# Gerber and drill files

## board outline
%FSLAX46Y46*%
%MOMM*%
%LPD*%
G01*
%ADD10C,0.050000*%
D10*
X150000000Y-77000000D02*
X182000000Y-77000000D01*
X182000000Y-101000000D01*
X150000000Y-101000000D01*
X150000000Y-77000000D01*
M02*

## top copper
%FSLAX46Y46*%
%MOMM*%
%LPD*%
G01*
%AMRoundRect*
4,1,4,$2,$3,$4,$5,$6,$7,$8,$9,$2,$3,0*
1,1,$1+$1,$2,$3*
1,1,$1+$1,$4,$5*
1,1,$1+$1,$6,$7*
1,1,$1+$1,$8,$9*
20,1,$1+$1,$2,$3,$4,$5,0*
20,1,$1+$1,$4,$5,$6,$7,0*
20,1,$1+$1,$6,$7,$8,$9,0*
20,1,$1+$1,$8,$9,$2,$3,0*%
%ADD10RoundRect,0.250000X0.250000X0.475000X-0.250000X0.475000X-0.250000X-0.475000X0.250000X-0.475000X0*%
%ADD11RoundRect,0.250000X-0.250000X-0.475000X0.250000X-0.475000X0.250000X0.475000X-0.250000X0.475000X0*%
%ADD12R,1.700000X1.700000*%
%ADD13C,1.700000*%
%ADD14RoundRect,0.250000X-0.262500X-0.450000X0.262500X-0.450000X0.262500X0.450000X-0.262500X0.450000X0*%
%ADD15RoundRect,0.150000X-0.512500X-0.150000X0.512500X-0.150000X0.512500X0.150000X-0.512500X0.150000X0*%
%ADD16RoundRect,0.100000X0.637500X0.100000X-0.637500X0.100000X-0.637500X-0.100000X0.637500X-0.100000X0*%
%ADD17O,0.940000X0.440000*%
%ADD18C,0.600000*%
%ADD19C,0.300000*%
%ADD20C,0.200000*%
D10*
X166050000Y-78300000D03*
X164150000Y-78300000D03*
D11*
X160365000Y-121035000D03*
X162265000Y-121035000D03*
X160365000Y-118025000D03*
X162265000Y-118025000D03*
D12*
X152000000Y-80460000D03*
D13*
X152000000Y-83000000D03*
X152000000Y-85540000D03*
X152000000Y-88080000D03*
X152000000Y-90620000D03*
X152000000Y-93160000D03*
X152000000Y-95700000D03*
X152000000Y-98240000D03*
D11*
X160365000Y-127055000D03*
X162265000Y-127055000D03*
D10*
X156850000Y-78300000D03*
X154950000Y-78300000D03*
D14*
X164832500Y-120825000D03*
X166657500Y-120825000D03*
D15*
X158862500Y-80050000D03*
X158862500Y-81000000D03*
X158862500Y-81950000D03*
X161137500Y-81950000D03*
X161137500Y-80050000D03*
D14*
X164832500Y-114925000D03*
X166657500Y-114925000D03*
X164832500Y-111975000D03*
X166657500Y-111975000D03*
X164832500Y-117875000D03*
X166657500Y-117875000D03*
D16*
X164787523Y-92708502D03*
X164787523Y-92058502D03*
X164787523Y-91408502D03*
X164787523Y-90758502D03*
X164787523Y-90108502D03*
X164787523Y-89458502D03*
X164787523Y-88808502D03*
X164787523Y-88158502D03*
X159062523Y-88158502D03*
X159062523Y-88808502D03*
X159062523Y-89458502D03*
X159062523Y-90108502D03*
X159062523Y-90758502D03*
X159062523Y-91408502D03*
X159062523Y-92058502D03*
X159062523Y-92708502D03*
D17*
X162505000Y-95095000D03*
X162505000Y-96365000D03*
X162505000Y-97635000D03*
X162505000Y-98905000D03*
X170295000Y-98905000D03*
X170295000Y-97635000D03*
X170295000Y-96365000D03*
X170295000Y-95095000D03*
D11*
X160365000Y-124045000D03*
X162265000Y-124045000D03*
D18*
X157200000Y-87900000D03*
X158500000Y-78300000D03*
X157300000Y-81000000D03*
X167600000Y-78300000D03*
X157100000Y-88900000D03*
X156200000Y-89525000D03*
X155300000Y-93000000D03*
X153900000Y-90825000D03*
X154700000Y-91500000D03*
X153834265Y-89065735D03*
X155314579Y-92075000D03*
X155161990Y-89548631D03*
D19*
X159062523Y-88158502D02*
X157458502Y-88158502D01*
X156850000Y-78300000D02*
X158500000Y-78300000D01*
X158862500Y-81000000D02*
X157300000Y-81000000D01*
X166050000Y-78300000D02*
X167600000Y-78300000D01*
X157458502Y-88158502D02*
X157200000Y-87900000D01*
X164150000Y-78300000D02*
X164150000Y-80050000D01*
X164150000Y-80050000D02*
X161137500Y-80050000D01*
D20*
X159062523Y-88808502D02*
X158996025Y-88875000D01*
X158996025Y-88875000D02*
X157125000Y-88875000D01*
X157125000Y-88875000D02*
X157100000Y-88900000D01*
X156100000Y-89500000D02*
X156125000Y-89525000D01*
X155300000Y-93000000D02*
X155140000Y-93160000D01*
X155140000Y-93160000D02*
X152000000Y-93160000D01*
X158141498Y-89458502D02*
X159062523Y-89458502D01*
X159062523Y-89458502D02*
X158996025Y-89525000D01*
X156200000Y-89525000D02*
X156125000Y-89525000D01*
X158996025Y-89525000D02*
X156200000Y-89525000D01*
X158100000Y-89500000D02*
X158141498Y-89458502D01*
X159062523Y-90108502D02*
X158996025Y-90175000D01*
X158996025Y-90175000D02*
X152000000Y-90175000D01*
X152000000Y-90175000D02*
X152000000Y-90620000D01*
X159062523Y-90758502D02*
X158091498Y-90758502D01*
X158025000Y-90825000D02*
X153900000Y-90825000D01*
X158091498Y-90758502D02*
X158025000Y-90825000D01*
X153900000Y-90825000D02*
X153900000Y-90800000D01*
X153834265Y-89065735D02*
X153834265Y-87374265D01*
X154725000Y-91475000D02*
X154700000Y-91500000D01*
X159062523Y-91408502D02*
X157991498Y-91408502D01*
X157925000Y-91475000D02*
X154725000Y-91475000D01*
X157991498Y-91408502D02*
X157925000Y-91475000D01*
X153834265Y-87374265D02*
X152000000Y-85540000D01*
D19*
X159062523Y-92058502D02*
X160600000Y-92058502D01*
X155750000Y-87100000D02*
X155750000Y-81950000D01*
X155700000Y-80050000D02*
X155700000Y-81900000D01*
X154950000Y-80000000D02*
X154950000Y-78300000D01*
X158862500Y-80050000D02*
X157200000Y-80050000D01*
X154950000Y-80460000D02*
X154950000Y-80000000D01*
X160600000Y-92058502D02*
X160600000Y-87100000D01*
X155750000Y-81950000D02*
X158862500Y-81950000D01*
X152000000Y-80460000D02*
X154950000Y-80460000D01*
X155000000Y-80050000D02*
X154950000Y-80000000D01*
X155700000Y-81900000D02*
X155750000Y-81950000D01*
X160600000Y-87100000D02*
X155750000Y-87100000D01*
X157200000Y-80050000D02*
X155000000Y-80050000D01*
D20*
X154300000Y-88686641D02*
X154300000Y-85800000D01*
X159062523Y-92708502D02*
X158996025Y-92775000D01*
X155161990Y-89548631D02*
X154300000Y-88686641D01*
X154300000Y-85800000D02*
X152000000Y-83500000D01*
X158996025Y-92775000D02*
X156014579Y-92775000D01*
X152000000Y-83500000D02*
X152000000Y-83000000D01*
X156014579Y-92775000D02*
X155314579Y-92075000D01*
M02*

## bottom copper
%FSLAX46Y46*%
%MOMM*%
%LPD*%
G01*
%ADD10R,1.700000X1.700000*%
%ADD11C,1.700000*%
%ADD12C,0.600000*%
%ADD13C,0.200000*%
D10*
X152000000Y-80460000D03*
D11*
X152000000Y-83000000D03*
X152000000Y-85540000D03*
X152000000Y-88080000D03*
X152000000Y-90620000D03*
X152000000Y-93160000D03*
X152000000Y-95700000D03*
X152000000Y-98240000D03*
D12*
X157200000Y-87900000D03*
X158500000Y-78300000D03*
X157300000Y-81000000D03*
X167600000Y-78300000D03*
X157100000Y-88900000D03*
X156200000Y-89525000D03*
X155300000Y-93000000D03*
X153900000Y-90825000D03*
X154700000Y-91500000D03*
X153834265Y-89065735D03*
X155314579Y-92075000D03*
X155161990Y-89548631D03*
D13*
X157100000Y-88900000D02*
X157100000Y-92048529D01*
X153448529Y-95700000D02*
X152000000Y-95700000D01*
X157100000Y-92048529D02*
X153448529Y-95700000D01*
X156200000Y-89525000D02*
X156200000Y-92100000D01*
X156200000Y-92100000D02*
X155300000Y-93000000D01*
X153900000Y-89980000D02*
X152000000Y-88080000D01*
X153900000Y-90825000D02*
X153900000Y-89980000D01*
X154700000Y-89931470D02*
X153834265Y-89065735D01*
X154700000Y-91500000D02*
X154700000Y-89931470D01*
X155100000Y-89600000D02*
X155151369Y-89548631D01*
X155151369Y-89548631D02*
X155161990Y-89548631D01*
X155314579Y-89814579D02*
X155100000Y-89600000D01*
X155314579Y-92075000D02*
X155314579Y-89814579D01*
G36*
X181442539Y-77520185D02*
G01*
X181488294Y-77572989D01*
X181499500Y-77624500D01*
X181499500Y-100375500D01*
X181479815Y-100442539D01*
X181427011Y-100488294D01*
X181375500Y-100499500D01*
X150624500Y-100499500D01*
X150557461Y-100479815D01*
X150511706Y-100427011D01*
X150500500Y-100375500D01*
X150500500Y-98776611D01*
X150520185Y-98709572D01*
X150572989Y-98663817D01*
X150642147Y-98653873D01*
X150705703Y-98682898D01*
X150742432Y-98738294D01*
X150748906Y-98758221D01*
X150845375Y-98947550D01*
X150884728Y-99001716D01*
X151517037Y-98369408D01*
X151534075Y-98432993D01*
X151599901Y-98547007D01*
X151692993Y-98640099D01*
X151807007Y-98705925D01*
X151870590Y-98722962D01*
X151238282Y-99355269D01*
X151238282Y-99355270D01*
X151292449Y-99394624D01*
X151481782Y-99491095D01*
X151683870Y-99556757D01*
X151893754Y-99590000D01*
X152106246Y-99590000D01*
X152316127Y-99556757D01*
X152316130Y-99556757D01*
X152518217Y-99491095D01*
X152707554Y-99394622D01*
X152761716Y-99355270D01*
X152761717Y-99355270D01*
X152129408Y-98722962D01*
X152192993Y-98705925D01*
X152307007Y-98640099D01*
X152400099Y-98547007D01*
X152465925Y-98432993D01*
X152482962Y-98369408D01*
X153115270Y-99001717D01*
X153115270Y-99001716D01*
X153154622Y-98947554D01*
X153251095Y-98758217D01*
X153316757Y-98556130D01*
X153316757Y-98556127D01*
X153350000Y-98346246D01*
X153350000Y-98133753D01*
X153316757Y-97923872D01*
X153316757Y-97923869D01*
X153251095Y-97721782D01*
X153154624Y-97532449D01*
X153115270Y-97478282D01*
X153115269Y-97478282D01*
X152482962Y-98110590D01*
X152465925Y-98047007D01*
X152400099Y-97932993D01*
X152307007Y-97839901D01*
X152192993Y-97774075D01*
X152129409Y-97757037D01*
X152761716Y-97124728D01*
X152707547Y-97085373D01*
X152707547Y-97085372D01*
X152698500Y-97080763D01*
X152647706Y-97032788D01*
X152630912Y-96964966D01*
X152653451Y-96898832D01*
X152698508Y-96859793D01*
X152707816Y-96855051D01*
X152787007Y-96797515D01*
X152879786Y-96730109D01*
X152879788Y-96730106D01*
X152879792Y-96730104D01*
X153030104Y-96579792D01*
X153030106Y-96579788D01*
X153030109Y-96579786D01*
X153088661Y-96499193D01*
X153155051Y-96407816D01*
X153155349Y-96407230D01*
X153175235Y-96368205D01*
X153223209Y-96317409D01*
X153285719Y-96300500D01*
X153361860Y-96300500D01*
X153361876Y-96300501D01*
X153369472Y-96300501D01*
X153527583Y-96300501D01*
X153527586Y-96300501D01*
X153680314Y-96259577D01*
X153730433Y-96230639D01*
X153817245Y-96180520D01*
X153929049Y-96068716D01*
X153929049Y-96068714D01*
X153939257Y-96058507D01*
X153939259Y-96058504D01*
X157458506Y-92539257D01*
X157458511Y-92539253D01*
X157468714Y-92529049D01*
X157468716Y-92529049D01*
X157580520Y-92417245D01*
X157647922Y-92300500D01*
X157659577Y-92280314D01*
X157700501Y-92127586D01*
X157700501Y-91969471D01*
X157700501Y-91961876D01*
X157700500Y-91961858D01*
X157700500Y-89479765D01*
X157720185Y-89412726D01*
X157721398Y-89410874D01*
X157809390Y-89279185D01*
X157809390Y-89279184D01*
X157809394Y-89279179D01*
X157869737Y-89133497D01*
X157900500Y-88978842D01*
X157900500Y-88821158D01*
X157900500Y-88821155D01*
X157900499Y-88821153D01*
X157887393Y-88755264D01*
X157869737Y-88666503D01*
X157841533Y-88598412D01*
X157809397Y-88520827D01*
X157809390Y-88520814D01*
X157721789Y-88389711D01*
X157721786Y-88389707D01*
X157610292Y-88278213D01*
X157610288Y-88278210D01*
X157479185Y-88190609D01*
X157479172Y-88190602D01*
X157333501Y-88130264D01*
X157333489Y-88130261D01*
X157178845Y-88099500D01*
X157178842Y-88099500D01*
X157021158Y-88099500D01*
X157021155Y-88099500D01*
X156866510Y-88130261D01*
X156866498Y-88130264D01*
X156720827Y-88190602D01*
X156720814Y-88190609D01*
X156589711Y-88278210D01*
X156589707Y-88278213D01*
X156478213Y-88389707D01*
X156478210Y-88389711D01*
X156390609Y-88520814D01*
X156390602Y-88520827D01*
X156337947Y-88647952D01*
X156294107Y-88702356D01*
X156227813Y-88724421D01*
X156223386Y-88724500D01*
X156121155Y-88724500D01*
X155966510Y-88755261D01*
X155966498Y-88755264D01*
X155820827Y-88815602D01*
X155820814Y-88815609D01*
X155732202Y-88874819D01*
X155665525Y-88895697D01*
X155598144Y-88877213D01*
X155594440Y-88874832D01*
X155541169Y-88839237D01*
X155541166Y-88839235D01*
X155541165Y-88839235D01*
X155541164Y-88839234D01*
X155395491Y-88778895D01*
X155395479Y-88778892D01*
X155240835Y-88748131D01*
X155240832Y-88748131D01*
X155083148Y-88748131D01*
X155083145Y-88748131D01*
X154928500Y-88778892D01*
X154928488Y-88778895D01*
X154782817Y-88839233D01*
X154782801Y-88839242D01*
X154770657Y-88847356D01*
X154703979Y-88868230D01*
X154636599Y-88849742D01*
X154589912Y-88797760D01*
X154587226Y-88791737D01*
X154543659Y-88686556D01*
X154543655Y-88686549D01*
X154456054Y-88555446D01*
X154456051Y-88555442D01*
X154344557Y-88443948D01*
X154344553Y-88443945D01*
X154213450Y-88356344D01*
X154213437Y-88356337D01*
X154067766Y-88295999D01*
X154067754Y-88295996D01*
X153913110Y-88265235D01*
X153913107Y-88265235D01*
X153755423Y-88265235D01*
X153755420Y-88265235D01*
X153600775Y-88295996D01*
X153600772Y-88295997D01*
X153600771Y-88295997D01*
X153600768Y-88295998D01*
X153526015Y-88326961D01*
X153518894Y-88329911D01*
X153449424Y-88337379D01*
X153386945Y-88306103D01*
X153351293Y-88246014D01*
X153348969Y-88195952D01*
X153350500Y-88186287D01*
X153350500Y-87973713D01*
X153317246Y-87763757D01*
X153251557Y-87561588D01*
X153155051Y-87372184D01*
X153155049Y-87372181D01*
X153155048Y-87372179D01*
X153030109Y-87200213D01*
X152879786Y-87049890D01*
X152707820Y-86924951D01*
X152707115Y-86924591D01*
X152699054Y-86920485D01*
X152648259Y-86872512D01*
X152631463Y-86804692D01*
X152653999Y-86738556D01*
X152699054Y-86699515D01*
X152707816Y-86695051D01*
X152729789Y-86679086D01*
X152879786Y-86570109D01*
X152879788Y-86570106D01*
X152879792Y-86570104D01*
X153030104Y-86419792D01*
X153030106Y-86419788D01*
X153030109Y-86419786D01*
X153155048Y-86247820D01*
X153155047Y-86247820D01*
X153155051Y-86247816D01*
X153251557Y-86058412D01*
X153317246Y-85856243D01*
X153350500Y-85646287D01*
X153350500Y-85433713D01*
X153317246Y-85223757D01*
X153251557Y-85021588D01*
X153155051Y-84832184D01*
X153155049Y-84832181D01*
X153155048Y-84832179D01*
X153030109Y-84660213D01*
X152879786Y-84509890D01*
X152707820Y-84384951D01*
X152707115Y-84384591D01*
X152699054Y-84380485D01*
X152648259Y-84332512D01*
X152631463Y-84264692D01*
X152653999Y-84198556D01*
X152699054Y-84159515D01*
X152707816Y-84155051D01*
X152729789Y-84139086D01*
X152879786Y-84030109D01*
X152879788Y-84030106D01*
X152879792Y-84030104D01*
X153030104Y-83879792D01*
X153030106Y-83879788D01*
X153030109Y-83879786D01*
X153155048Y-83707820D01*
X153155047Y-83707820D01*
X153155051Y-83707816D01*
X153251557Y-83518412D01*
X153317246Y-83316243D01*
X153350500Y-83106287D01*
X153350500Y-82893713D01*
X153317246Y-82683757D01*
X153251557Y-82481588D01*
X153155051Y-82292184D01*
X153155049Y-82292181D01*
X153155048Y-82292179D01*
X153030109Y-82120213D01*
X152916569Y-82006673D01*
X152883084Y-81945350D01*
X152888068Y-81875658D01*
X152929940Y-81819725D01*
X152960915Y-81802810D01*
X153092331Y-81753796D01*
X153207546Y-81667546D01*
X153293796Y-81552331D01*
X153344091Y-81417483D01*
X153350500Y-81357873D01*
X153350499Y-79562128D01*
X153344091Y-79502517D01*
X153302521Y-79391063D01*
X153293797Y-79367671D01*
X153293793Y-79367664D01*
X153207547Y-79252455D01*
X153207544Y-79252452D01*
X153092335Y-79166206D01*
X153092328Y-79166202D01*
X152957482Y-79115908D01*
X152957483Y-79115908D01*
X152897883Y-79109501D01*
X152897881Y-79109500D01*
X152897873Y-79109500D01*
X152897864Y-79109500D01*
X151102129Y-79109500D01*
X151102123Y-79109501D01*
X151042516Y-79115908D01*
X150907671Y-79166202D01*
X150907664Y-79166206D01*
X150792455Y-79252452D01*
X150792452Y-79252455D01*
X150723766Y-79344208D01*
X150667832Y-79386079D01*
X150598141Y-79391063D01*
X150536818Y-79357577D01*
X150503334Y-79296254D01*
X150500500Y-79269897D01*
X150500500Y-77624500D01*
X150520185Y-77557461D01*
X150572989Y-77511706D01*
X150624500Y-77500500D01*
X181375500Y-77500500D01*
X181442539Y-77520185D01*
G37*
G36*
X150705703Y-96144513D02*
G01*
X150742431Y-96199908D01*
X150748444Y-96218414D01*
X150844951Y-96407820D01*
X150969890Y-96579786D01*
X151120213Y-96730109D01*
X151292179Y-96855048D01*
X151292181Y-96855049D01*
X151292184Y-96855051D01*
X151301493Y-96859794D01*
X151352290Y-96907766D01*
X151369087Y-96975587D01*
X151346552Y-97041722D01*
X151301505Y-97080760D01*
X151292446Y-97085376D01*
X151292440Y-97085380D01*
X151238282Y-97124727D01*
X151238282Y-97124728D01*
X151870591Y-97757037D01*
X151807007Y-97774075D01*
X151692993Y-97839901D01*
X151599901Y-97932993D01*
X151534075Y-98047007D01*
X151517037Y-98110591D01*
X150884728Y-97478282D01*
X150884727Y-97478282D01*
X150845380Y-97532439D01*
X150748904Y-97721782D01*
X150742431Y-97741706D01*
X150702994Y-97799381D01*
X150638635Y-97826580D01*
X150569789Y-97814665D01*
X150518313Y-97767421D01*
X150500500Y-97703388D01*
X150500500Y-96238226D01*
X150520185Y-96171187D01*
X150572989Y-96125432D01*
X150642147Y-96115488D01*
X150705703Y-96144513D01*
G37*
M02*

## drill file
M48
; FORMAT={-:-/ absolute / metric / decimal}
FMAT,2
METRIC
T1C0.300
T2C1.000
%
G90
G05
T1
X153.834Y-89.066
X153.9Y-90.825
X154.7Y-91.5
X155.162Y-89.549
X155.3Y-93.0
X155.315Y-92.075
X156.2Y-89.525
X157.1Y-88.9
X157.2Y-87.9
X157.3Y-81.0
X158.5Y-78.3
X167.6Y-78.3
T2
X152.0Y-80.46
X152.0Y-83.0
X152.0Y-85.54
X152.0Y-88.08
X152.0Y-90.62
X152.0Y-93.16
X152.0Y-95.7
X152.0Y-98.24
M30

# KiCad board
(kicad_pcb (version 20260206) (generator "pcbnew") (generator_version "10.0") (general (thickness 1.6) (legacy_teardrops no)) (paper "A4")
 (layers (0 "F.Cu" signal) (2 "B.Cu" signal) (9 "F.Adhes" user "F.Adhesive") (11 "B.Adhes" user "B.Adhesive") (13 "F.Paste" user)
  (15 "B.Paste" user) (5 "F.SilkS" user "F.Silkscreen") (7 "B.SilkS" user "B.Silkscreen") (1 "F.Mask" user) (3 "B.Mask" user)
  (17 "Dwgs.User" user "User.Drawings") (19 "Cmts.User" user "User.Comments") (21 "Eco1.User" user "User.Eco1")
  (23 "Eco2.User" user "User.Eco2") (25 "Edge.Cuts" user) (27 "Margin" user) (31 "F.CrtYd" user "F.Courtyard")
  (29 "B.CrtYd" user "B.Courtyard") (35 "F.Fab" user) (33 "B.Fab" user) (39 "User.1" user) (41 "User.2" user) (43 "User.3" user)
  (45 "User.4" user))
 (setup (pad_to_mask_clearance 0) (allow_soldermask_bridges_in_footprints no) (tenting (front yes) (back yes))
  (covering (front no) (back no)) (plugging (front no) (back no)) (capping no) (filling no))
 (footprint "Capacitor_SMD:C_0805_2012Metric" (layer "F.Cu") (at 165.1 78.3 180)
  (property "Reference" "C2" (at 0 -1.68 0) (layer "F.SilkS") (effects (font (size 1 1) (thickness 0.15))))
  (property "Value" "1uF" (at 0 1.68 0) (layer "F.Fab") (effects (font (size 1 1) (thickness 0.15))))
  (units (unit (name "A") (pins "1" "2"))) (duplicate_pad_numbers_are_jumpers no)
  (pad "1" smd roundrect (at -0.95 0 180) (size 1 1.45) (layers "F.Cu" "F.Mask" "F.Paste") (roundrect_rratio 0.25) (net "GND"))
  (pad "2" smd roundrect (at 0.95 0 180) (size 1 1.45) (layers "F.Cu" "F.Mask" "F.Paste") (roundrect_rratio 0.25) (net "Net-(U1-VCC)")))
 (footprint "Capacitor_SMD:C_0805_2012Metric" (layer "F.Cu") (at 161.315 121.035)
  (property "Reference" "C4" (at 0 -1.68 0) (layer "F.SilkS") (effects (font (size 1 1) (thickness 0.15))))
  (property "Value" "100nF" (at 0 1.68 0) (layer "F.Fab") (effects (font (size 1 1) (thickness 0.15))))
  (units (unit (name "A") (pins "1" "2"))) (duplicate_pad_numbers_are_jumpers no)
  (pad "1" smd roundrect (at -0.95 0) (size 1 1.45) (layers "F.Cu" "F.Mask" "F.Paste") (roundrect_rratio 0.25) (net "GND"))
  (pad "2" smd roundrect (at 0.95 0) (size 1 1.45) (layers "F.Cu" "F.Mask" "F.Paste") (roundrect_rratio 0.25) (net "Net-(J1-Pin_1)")))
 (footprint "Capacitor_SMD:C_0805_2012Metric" (layer "F.Cu") (at 161.315 118.025)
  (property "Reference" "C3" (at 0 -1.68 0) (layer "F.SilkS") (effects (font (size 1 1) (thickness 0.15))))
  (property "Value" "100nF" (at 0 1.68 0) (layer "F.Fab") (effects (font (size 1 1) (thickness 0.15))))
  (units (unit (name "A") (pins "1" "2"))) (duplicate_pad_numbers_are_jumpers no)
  (pad "1" smd roundrect (at -0.95 0) (size 1 1.45) (layers "F.Cu" "F.Mask" "F.Paste") (roundrect_rratio 0.25) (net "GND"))
  (pad "2" smd roundrect (at 0.95 0) (size 1 1.45) (layers "F.Cu" "F.Mask" "F.Paste") (roundrect_rratio 0.25) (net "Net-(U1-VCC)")))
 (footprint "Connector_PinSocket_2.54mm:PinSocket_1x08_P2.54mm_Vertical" (layer "F.Cu") (at 152 80.46)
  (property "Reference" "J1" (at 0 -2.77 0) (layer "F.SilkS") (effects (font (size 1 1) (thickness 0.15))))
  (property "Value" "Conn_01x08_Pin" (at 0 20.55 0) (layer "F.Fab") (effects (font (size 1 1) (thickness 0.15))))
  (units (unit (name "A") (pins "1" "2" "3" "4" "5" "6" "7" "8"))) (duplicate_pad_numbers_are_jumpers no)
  (pad "1" thru_hole rect (at 0 0) (size 1.7 1.7) (drill 1) (layers "*.Cu" "*.Mask") (remove_unused_layers no) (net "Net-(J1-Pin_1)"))
  (pad "2" thru_hole circle (at 0 2.54) (size 1.7 1.7) (drill 1) (layers "*.Cu" "*.Mask") (remove_unused_layers no) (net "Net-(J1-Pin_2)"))
  (pad "3" thru_hole circle (at 0 5.08) (size 1.7 1.7) (drill 1) (layers "*.Cu" "*.Mask") (remove_unused_layers no) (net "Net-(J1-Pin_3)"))
  (pad "4" thru_hole circle (at 0 7.62) (size 1.7 1.7) (drill 1) (layers "*.Cu" "*.Mask") (remove_unused_layers no) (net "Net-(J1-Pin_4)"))
  (pad "5" thru_hole circle (at 0 10.16) (size 1.7 1.7) (drill 1) (layers "*.Cu" "*.Mask") (remove_unused_layers no) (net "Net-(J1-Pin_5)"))
  (pad "6" thru_hole circle (at 0 12.7) (size 1.7 1.7) (drill 1) (layers "*.Cu" "*.Mask") (remove_unused_layers no) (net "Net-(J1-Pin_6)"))
  (pad "7" thru_hole circle (at 0 15.24) (size 1.7 1.7) (drill 1) (layers "*.Cu" "*.Mask") (remove_unused_layers no) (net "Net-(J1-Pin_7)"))
  (pad "8" thru_hole circle (at 0 17.78) (size 1.7 1.7) (drill 1) (layers "*.Cu" "*.Mask") (remove_unused_layers no) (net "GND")))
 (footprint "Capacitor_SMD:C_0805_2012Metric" (layer "F.Cu") (at 161.315 127.055)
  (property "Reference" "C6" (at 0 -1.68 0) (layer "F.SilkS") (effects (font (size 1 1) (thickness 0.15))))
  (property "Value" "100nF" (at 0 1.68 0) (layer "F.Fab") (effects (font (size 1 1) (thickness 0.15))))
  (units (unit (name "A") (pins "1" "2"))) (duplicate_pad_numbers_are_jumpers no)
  (pad "1" smd roundrect (at -0.95 0) (size 1 1.45) (layers "F.Cu" "F.Mask" "F.Paste") (roundrect_rratio 0.25) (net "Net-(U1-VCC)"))
  (pad "2" smd roundrect (at 0.95 0) (size 1 1.45) (layers "F.Cu" "F.Mask" "F.Paste") (roundrect_rratio 0.25) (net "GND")))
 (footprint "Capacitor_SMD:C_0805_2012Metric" (layer "F.Cu") (at 155.9 78.3 180)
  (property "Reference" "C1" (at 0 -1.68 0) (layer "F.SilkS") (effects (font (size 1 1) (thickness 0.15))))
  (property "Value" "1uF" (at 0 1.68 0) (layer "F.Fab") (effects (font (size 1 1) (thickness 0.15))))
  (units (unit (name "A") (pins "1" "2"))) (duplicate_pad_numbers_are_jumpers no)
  (pad "1" smd roundrect (at -0.95 0 180) (size 1 1.45) (layers "F.Cu" "F.Mask" "F.Paste") (roundrect_rratio 0.25) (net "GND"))
  (pad "2" smd roundrect (at 0.95 0 180) (size 1 1.45) (layers "F.Cu" "F.Mask" "F.Paste") (roundrect_rratio 0.25) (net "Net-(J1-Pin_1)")))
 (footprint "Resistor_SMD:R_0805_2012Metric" (layer "F.Cu") (at 165.745 120.825)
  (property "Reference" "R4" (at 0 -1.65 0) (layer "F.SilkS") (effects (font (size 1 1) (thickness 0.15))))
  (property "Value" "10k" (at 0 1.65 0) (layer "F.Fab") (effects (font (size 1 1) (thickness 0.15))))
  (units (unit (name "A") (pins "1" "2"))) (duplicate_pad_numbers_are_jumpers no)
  (pad "1" smd roundrect (at -0.9125 0) (size 1.025 1.4) (layers "F.Cu" "F.Mask" "F.Paste") (roundrect_rratio 0.243902) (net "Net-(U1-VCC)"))
  (pad "2" smd roundrect (at 0.9125 0) (size 1.025 1.4) (layers "F.Cu" "F.Mask" "F.Paste") (roundrect_rratio 0.243902)
   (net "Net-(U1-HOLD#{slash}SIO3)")))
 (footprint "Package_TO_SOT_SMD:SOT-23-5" (layer "F.Cu") (at 160 81)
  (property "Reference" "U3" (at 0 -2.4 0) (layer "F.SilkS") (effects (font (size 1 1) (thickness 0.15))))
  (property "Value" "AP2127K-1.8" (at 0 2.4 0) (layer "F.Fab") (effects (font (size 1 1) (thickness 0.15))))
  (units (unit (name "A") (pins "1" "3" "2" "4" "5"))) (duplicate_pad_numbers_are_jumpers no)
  (pad "1" smd roundrect (at -1.1375 -0.95) (size 1.325 0.6) (layers "F.Cu" "F.Mask" "F.Paste") (roundrect_rratio 0.25)
   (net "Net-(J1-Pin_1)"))
  (pad "2" smd roundrect (at -1.1375 0) (size 1.325 0.6) (layers "F.Cu" "F.Mask" "F.Paste") (roundrect_rratio 0.25) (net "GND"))
  (pad "3" smd roundrect (at -1.1375 0.95) (size 1.325 0.6) (layers "F.Cu" "F.Mask" "F.Paste") (roundrect_rratio 0.25)
   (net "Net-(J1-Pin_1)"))
  (pad "4" smd roundrect (at 1.1375 0.95) (size 1.325 0.6) (layers "F.Cu" "F.Mask" "F.Paste") (roundrect_rratio 0.25)
   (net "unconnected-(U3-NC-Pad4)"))
  (pad "5" smd roundrect (at 1.1375 -0.95) (size 1.325 0.6) (layers "F.Cu" "F.Mask" "F.Paste") (roundrect_rratio 0.25) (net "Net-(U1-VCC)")))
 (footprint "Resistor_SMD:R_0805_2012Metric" (layer "F.Cu") (at 165.745 114.925)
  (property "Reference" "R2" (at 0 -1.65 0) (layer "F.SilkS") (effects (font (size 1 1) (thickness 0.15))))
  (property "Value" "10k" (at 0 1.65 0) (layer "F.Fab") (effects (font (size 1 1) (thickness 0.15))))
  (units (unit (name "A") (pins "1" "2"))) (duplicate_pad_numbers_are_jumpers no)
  (pad "1" smd roundrect (at -0.9125 0) (size 1.025 1.4) (layers "F.Cu" "F.Mask" "F.Paste") (roundrect_rratio 0.243902) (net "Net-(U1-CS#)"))
  (pad "2" smd roundrect (at 0.9125 0) (size 1.025 1.4) (layers "F.Cu" "F.Mask" "F.Paste") (roundrect_rratio 0.243902) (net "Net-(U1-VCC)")))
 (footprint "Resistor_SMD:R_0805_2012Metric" (layer "F.Cu") (at 165.745 111.975)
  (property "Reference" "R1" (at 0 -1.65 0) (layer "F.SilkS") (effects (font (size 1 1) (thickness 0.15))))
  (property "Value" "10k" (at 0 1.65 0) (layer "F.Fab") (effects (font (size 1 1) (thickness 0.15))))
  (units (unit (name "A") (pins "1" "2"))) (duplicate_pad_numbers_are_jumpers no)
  (pad "1" smd roundrect (at -0.9125 0) (size 1.025 1.4) (layers "F.Cu" "F.Mask" "F.Paste") (roundrect_rratio 0.243902) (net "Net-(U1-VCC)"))
  (pad "2" smd roundrect (at 0.9125 0) (size 1.025 1.4) (layers "F.Cu" "F.Mask" "F.Paste") (roundrect_rratio 0.243902) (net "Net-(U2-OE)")))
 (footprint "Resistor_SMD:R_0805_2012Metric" (layer "F.Cu") (at 165.745 117.875)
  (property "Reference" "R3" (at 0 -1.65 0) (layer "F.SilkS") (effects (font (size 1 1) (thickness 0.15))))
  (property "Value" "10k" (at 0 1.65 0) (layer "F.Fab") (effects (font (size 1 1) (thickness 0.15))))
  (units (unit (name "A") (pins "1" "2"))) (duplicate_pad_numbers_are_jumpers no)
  (pad "1" smd roundrect (at -0.9125 0) (size 1.025 1.4) (layers "F.Cu" "F.Mask" "F.Paste") (roundrect_rratio 0.243902) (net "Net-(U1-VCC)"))
  (pad "2" smd roundrect (at 0.9125 0) (size 1.025 1.4) (layers "F.Cu" "F.Mask" "F.Paste") (roundrect_rratio 0.243902)
   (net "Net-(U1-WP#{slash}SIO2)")))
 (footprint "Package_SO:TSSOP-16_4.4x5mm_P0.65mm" (layer "F.Cu") (at 161.925023 90.433502 180)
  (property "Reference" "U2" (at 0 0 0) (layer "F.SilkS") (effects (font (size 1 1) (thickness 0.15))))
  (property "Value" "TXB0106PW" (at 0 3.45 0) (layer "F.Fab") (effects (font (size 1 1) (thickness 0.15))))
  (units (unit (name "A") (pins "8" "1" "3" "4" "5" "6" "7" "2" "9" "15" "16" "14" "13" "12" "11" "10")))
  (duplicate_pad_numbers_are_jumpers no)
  (pad "1" smd roundrect (at -2.8625 -2.275 180) (size 1.475 0.4) (layers "F.Cu" "F.Mask" "F.Paste") (roundrect_rratio 0.25)
   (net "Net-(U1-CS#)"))
  (pad "2" smd roundrect (at -2.8625 -1.625 180) (size 1.475 0.4) (layers "F.Cu" "F.Mask" "F.Paste") (roundrect_rratio 0.25)
   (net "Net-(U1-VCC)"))
  (pad "3" smd roundrect (at -2.8625 -0.975 180) (size 1.475 0.4) (layers "F.Cu" "F.Mask" "F.Paste") (roundrect_rratio 0.25)
   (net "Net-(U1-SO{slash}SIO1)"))
  (pad "4" smd roundrect (at -2.8625 -0.325 180) (size 1.475 0.4) (layers "F.Cu" "F.Mask" "F.Paste") (roundrect_rratio 0.25)
   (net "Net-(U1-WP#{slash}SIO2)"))
  (pad "5" smd roundrect (at -2.8625 0.325 180) (size 1.475 0.4) (layers "F.Cu" "F.Mask" "F.Paste") (roundrect_rratio 0.25)
   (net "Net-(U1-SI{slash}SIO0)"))
  (pad "6" smd roundrect (at -2.8625 0.975 180) (size 1.475 0.4) (layers "F.Cu" "F.Mask" "F.Paste") (roundrect_rratio 0.25)
   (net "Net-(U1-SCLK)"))
  (pad "7" smd roundrect (at -2.8625 1.625 180) (size 1.475 0.4) (layers "F.Cu" "F.Mask" "F.Paste") (roundrect_rratio 0.25)
   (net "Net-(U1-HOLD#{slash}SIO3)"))
  (pad "8" smd roundrect (at -2.8625 2.275 180) (size 1.475 0.4) (layers "F.Cu" "F.Mask" "F.Paste") (roundrect_rratio 0.25)
   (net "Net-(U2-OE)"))
  (pad "9" smd roundrect (at 2.8625 2.275 180) (size 1.475 0.4) (layers "F.Cu" "F.Mask" "F.Paste") (roundrect_rratio 0.25) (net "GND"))
  (pad "10" smd roundrect (at 2.8625 1.625 180) (size 1.475 0.4) (layers "F.Cu" "F.Mask" "F.Paste") (roundrect_rratio 0.25)
   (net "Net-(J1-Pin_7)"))
  (pad "11" smd roundrect (at 2.8625 0.975 180) (size 1.475 0.4) (layers "F.Cu" "F.Mask" "F.Paste") (roundrect_rratio 0.25)
   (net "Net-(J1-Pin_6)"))
  (pad "12" smd roundrect (at 2.8625 0.325 180) (size 1.475 0.4) (layers "F.Cu" "F.Mask" "F.Paste") (roundrect_rratio 0.25)
   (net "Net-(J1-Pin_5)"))
  (pad "13" smd roundrect (at 2.8625 -0.325 180) (size 1.475 0.4) (layers "F.Cu" "F.Mask" "F.Paste") (roundrect_rratio 0.25)
   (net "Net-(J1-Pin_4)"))
  (pad "14" smd roundrect (at 2.8625 -0.975 180) (size 1.475 0.4) (layers "F.Cu" "F.Mask" "F.Paste") (roundrect_rratio 0.25)
   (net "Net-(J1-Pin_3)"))
  (pad "15" smd roundrect (at 2.8625 -1.625 180) (size 1.475 0.4) (layers "F.Cu" "F.Mask" "F.Paste") (roundrect_rratio 0.25)
   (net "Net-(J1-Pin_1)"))
  (pad "16" smd roundrect (at 2.8625 -2.275 180) (size 1.475 0.4) (layers "F.Cu" "F.Mask" "F.Paste") (roundrect_rratio 0.25)
   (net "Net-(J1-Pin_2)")))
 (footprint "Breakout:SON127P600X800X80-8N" (layer "F.Cu") (at 166.4 97)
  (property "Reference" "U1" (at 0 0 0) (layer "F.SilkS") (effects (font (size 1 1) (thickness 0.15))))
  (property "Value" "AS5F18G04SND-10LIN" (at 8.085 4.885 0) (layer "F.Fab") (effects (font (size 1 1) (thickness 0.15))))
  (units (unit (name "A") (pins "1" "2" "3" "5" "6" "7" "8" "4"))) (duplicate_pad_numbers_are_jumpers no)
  (pad "1" smd oval (at -3.895 -1.905) (size 0.94 0.44) (layers "F.Cu" "F.Mask" "F.Paste") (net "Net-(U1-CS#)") (solder_mask_margin 0.102))
  (pad "2" smd oval (at -3.895 -0.635) (size 0.94 0.44) (layers "F.Cu" "F.Mask" "F.Paste") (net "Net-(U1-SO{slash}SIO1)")
   (solder_mask_margin 0.102))
  (pad "3" smd oval (at -3.895 0.635) (size 0.94 0.44) (layers "F.Cu" "F.Mask" "F.Paste") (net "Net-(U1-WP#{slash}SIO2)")
   (solder_mask_margin 0.102))
  (pad "4" smd oval (at -3.895 1.905) (size 0.94 0.44) (layers "F.Cu" "F.Mask" "F.Paste") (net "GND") (solder_mask_margin 0.102))
  (pad "5" smd oval (at 3.895 1.905) (size 0.94 0.44) (layers "F.Cu" "F.Mask" "F.Paste") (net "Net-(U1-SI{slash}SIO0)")
   (solder_mask_margin 0.102))
  (pad "6" smd oval (at 3.895 0.635) (size 0.94 0.44) (layers "F.Cu" "F.Mask" "F.Paste") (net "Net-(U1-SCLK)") (solder_mask_margin 0.102))
  (pad "7" smd oval (at 3.895 -0.635) (size 0.94 0.44) (layers "F.Cu" "F.Mask" "F.Paste") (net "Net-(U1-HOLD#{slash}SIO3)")
   (solder_mask_margin 0.102))
  (pad "8" smd oval (at 3.895 -1.905) (size 0.94 0.44) (layers "F.Cu" "F.Mask" "F.Paste") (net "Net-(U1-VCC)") (solder_mask_margin 0.102)))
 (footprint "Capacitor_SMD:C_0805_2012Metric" (layer "F.Cu") (at 161.315 124.045)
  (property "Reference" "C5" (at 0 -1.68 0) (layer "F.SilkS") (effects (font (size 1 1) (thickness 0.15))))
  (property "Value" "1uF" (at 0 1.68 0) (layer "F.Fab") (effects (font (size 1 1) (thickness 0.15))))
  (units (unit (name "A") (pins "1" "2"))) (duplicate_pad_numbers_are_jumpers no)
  (pad "1" smd roundrect (at -0.95 0) (size 1 1.45) (layers "F.Cu" "F.Mask" "F.Paste") (roundrect_rratio 0.25) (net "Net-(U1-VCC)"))
  (pad "2" smd roundrect (at 0.95 0) (size 1 1.45) (layers "F.Cu" "F.Mask" "F.Paste") (roundrect_rratio 0.25) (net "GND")))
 (gr_rect (start 150 77) (end 182 101) (stroke (width 0.05) (type default)) (fill no) (layer "Edge.Cuts"))
 (segment (start 159.062523 88.158502) (end 157.458502 88.158502) (width 0.3) (layer "F.Cu") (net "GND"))
 (segment (start 156.85 78.3) (end 158.5 78.3) (width 0.3) (layer "F.Cu") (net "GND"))
 (segment (start 158.8625 81) (end 157.3 81) (width 0.3) (layer "F.Cu") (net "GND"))
 (segment (start 166.05 78.3) (end 167.6 78.3) (width 0.3) (layer "F.Cu") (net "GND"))
 (segment (start 157.458502 88.158502) (end 157.2 87.9) (width 0.3) (layer "F.Cu") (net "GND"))
 (via (at 157.2 87.9) (size 0.6) (drill 0.3) (layers "F.Cu" "B.Cu") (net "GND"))
 (via (at 158.5 78.3) (size 0.6) (drill 0.3) (layers "F.Cu" "B.Cu") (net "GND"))
 (via (at 157.3 81) (size 0.6) (drill 0.3) (layers "F.Cu" "B.Cu") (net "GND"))
 (via (at 167.6 78.3) (size 0.6) (drill 0.3) (layers "F.Cu" "B.Cu") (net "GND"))
 (segment (start 164.15 78.3) (end 164.15 80.05) (width 0.3) (layer "F.Cu") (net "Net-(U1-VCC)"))
 (segment (start 164.15 80.05) (end 161.1375 80.05) (width 0.3) (layer "F.Cu") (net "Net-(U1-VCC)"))
 (segment (start 159.062523 88.808502) (end 158.996025 88.875) (width 0.2) (layer "F.Cu") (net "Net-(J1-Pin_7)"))
 (segment (start 158.996025 88.875) (end 157.125 88.875) (width 0.2) (layer "F.Cu") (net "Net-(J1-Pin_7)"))
 (segment (start 157.125 88.875) (end 157.1 88.9) (width 0.2) (layer "F.Cu") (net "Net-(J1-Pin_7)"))
 (via (at 157.1 88.9) (size 0.6) (drill 0.3) (layers "F.Cu" "B.Cu") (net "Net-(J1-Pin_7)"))
 (segment (start 157.1 88.9) (end 157.1 92.048529) (width 0.2) (layer "B.Cu") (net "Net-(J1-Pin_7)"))
 (segment (start 153.448529 95.7) (end 152 95.7) (width 0.2) (layer "B.Cu") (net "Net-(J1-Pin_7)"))
 (segment (start 157.1 92.048529) (end 153.448529 95.7) (width 0.2) (layer "B.Cu") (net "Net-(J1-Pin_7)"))
 (segment (start 156.1 89.5) (end 156.125 89.525) (width 0.2) (layer "F.Cu") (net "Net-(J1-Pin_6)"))
 (segment (start 155.3 93) (end 155.14 93.16) (width 0.2) (layer "F.Cu") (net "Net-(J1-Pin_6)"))
 (segment (start 155.14 93.16) (end 152 93.16) (width 0.2) (layer "F.Cu") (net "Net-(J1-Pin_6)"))
 (segment (start 158.141498 89.458502) (end 159.062523 89.458502) (width 0.2) (layer "F.Cu") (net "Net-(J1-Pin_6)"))
 (segment (start 159.062523 89.458502) (end 158.996025 89.525) (width 0.2) (layer "F.Cu") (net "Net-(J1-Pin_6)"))
 (segment (start 156.2 89.525) (end 156.125 89.525) (width 0.2) (layer "F.Cu") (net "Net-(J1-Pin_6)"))
 (segment (start 158.996025 89.525) (end 156.2 89.525) (width 0.2) (layer "F.Cu") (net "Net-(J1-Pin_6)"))
 (segment (start 158.1 89.5) (end 158.141498 89.458502) (width 0.2) (layer "F.Cu") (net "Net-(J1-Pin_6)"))
 (via (at 156.2 89.525) (size 0.6) (drill 0.3) (layers "F.Cu" "B.Cu") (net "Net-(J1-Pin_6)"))
 (via (at 155.3 93) (size 0.6) (drill 0.3) (layers "F.Cu" "B.Cu") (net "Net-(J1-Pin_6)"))
 (segment (start 156.2 89.525) (end 156.2 92.1) (width 0.2) (layer "B.Cu") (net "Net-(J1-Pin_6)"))
 (segment (start 156.2 92.1) (end 155.3 93) (width 0.2) (layer "B.Cu") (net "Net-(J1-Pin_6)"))
 (segment (start 159.062523 90.108502) (end 158.996025 90.175) (width 0.2) (layer "F.Cu") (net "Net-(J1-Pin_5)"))
 (segment (start 158.996025 90.175) (end 152 90.175) (width 0.2) (layer "F.Cu") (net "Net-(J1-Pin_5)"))
 (segment (start 152 90.175) (end 152 90.62) (width 0.2) (layer "F.Cu") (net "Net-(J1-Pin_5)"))
 (segment (start 159.062523 90.758502) (end 158.091498 90.758502) (width 0.2) (layer "F.Cu") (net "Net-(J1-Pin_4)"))
 (segment (start 158.025 90.825) (end 153.9 90.825) (width 0.2) (layer "F.Cu") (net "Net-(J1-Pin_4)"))
 (segment (start 158.091498 90.758502) (end 158.025 90.825) (width 0.2) (layer "F.Cu") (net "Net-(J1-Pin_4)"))
 (segment (start 153.9 90.825) (end 153.9 90.8) (width 0.2) (layer "F.Cu") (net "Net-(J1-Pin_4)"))
 (via (at 153.9 90.825) (size 0.6) (drill 0.3) (layers "F.Cu" "B.Cu") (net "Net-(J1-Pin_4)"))
 (segment (start 153.9 89.98) (end 152 88.08) (width 0.2) (layer "B.Cu") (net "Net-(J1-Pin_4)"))
 (segment (start 153.9 90.825) (end 153.9 89.98) (width 0.2) (layer "B.Cu") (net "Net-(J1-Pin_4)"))
 (segment (start 153.834265 89.065735) (end 153.834265 87.374265) (width 0.2) (layer "F.Cu") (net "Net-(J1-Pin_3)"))
 (segment (start 154.725 91.475) (end 154.7 91.5) (width 0.2) (layer "F.Cu") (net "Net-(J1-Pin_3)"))
 (segment (start 159.062523 91.408502) (end 157.991498 91.408502) (width 0.2) (layer "F.Cu") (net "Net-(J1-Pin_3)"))
 (segment (start 157.925 91.475) (end 154.725 91.475) (width 0.2) (layer "F.Cu") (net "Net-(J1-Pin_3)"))
 (segment (start 157.991498 91.408502) (end 157.925 91.475) (width 0.2) (layer "F.Cu") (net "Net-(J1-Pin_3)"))
 (segment (start 153.834265 87.374265) (end 152 85.54) (width 0.2) (layer "F.Cu") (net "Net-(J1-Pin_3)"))
 (via (at 154.7 91.5) (size 0.6) (drill 0.3) (layers "F.Cu" "B.Cu") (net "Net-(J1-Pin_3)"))
 (via (at 153.834265 89.065735) (size 0.6) (drill 0.3) (layers "F.Cu" "B.Cu") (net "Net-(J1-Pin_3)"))
 (segment (start 154.7 89.93147) (end 153.834265 89.065735) (width 0.2) (layer "B.Cu") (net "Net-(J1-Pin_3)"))
 (segment (start 154.7 91.5) (end 154.7 89.93147) (width 0.2) (layer "B.Cu") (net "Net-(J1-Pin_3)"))
 (segment (start 159.062523 92.058502) (end 160.6 92.058502) (width 0.3) (layer "F.Cu") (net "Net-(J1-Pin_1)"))
 (segment (start 155.75 87.1) (end 155.75 81.95) (width 0.3) (layer "F.Cu") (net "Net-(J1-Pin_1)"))
 (segment (start 155.7 80.05) (end 155.7 81.9) (width 0.3) (layer "F.Cu") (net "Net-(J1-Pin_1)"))
 (segment (start 154.95 80) (end 154.95 78.3) (width 0.3) (layer "F.Cu") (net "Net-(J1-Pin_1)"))
 (segment (start 158.8625 80.05) (end 157.2 80.05) (width 0.3) (layer "F.Cu") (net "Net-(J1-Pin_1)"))
 (segment (start 154.95 80.46) (end 154.95 80) (width 0.3) (layer "F.Cu") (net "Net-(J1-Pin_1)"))
 (segment (start 160.6 92.058502) (end 160.6 87.1) (width 0.3) (layer "F.Cu") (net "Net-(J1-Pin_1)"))
 (segment (start 155.75 81.95) (end 158.8625 81.95) (width 0.3) (layer "F.Cu") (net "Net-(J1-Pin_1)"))
 (segment (start 152 80.46) (end 154.95 80.46) (width 0.3) (layer "F.Cu") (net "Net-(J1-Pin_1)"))
 (segment (start 155 80.05) (end 154.95 80) (width 0.3) (layer "F.Cu") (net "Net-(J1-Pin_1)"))
 (segment (start 155.7 81.9) (end 155.75 81.95) (width 0.3) (layer "F.Cu") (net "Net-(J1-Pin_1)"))
 (segment (start 160.6 87.1) (end 155.75 87.1) (width 0.3) (layer "F.Cu") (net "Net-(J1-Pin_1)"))
 (segment (start 157.2 80.05) (end 155 80.05) (width 0.3) (layer "F.Cu") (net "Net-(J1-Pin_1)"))
 (segment (start 154.3 88.686641) (end 154.3 85.8) (width 0.2) (layer "F.Cu") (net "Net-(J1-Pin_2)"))
 (segment (start 159.062523 92.708502) (end 158.996025 92.775) (width 0.2) (layer "F.Cu") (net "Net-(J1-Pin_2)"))
 (segment (start 155.16199 89.548631) (end 154.3 88.686641) (width 0.2) (layer "F.Cu") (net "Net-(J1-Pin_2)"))
 (segment (start 154.3 85.8) (end 152 83.5) (width 0.2) (layer "F.Cu") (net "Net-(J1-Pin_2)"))
 (segment (start 158.996025 92.775) (end 156.014579 92.775) (width 0.2) (layer "F.Cu") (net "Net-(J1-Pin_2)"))
 (segment (start 152 83.5) (end 152 83) (width 0.2) (layer "F.Cu") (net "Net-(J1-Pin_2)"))
 (segment (start 156.014579 92.775) (end 155.314579 92.075) (width 0.2) (layer "F.Cu") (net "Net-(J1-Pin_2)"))
 (via (at 155.314579 92.075) (size 0.6) (drill 0.3) (layers "F.Cu" "B.Cu") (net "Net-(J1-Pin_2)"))
 (via (at 155.16199 89.548631) (size 0.6) (drill 0.3) (layers "F.Cu" "B.Cu") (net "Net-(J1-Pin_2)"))
 (segment (start 155.1 89.6) (end 155.151369 89.548631) (width 0.2) (layer "B.Cu") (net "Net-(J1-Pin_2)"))
 (segment (start 155.151369 89.548631) (end 155.16199 89.548631) (width 0.2) (layer "B.Cu") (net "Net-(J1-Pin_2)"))
 (segment (start 155.314579 89.814579) (end 155.1 89.6) (width 0.2) (layer "B.Cu") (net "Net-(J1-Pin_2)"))
 (segment (start 155.314579 92.075) (end 155.314579 89.814579) (width 0.2) (layer "B.Cu") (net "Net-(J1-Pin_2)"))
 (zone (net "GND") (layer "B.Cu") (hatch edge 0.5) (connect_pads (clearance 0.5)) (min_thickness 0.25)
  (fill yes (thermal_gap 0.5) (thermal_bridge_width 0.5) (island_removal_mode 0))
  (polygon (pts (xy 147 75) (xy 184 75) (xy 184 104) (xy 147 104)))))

